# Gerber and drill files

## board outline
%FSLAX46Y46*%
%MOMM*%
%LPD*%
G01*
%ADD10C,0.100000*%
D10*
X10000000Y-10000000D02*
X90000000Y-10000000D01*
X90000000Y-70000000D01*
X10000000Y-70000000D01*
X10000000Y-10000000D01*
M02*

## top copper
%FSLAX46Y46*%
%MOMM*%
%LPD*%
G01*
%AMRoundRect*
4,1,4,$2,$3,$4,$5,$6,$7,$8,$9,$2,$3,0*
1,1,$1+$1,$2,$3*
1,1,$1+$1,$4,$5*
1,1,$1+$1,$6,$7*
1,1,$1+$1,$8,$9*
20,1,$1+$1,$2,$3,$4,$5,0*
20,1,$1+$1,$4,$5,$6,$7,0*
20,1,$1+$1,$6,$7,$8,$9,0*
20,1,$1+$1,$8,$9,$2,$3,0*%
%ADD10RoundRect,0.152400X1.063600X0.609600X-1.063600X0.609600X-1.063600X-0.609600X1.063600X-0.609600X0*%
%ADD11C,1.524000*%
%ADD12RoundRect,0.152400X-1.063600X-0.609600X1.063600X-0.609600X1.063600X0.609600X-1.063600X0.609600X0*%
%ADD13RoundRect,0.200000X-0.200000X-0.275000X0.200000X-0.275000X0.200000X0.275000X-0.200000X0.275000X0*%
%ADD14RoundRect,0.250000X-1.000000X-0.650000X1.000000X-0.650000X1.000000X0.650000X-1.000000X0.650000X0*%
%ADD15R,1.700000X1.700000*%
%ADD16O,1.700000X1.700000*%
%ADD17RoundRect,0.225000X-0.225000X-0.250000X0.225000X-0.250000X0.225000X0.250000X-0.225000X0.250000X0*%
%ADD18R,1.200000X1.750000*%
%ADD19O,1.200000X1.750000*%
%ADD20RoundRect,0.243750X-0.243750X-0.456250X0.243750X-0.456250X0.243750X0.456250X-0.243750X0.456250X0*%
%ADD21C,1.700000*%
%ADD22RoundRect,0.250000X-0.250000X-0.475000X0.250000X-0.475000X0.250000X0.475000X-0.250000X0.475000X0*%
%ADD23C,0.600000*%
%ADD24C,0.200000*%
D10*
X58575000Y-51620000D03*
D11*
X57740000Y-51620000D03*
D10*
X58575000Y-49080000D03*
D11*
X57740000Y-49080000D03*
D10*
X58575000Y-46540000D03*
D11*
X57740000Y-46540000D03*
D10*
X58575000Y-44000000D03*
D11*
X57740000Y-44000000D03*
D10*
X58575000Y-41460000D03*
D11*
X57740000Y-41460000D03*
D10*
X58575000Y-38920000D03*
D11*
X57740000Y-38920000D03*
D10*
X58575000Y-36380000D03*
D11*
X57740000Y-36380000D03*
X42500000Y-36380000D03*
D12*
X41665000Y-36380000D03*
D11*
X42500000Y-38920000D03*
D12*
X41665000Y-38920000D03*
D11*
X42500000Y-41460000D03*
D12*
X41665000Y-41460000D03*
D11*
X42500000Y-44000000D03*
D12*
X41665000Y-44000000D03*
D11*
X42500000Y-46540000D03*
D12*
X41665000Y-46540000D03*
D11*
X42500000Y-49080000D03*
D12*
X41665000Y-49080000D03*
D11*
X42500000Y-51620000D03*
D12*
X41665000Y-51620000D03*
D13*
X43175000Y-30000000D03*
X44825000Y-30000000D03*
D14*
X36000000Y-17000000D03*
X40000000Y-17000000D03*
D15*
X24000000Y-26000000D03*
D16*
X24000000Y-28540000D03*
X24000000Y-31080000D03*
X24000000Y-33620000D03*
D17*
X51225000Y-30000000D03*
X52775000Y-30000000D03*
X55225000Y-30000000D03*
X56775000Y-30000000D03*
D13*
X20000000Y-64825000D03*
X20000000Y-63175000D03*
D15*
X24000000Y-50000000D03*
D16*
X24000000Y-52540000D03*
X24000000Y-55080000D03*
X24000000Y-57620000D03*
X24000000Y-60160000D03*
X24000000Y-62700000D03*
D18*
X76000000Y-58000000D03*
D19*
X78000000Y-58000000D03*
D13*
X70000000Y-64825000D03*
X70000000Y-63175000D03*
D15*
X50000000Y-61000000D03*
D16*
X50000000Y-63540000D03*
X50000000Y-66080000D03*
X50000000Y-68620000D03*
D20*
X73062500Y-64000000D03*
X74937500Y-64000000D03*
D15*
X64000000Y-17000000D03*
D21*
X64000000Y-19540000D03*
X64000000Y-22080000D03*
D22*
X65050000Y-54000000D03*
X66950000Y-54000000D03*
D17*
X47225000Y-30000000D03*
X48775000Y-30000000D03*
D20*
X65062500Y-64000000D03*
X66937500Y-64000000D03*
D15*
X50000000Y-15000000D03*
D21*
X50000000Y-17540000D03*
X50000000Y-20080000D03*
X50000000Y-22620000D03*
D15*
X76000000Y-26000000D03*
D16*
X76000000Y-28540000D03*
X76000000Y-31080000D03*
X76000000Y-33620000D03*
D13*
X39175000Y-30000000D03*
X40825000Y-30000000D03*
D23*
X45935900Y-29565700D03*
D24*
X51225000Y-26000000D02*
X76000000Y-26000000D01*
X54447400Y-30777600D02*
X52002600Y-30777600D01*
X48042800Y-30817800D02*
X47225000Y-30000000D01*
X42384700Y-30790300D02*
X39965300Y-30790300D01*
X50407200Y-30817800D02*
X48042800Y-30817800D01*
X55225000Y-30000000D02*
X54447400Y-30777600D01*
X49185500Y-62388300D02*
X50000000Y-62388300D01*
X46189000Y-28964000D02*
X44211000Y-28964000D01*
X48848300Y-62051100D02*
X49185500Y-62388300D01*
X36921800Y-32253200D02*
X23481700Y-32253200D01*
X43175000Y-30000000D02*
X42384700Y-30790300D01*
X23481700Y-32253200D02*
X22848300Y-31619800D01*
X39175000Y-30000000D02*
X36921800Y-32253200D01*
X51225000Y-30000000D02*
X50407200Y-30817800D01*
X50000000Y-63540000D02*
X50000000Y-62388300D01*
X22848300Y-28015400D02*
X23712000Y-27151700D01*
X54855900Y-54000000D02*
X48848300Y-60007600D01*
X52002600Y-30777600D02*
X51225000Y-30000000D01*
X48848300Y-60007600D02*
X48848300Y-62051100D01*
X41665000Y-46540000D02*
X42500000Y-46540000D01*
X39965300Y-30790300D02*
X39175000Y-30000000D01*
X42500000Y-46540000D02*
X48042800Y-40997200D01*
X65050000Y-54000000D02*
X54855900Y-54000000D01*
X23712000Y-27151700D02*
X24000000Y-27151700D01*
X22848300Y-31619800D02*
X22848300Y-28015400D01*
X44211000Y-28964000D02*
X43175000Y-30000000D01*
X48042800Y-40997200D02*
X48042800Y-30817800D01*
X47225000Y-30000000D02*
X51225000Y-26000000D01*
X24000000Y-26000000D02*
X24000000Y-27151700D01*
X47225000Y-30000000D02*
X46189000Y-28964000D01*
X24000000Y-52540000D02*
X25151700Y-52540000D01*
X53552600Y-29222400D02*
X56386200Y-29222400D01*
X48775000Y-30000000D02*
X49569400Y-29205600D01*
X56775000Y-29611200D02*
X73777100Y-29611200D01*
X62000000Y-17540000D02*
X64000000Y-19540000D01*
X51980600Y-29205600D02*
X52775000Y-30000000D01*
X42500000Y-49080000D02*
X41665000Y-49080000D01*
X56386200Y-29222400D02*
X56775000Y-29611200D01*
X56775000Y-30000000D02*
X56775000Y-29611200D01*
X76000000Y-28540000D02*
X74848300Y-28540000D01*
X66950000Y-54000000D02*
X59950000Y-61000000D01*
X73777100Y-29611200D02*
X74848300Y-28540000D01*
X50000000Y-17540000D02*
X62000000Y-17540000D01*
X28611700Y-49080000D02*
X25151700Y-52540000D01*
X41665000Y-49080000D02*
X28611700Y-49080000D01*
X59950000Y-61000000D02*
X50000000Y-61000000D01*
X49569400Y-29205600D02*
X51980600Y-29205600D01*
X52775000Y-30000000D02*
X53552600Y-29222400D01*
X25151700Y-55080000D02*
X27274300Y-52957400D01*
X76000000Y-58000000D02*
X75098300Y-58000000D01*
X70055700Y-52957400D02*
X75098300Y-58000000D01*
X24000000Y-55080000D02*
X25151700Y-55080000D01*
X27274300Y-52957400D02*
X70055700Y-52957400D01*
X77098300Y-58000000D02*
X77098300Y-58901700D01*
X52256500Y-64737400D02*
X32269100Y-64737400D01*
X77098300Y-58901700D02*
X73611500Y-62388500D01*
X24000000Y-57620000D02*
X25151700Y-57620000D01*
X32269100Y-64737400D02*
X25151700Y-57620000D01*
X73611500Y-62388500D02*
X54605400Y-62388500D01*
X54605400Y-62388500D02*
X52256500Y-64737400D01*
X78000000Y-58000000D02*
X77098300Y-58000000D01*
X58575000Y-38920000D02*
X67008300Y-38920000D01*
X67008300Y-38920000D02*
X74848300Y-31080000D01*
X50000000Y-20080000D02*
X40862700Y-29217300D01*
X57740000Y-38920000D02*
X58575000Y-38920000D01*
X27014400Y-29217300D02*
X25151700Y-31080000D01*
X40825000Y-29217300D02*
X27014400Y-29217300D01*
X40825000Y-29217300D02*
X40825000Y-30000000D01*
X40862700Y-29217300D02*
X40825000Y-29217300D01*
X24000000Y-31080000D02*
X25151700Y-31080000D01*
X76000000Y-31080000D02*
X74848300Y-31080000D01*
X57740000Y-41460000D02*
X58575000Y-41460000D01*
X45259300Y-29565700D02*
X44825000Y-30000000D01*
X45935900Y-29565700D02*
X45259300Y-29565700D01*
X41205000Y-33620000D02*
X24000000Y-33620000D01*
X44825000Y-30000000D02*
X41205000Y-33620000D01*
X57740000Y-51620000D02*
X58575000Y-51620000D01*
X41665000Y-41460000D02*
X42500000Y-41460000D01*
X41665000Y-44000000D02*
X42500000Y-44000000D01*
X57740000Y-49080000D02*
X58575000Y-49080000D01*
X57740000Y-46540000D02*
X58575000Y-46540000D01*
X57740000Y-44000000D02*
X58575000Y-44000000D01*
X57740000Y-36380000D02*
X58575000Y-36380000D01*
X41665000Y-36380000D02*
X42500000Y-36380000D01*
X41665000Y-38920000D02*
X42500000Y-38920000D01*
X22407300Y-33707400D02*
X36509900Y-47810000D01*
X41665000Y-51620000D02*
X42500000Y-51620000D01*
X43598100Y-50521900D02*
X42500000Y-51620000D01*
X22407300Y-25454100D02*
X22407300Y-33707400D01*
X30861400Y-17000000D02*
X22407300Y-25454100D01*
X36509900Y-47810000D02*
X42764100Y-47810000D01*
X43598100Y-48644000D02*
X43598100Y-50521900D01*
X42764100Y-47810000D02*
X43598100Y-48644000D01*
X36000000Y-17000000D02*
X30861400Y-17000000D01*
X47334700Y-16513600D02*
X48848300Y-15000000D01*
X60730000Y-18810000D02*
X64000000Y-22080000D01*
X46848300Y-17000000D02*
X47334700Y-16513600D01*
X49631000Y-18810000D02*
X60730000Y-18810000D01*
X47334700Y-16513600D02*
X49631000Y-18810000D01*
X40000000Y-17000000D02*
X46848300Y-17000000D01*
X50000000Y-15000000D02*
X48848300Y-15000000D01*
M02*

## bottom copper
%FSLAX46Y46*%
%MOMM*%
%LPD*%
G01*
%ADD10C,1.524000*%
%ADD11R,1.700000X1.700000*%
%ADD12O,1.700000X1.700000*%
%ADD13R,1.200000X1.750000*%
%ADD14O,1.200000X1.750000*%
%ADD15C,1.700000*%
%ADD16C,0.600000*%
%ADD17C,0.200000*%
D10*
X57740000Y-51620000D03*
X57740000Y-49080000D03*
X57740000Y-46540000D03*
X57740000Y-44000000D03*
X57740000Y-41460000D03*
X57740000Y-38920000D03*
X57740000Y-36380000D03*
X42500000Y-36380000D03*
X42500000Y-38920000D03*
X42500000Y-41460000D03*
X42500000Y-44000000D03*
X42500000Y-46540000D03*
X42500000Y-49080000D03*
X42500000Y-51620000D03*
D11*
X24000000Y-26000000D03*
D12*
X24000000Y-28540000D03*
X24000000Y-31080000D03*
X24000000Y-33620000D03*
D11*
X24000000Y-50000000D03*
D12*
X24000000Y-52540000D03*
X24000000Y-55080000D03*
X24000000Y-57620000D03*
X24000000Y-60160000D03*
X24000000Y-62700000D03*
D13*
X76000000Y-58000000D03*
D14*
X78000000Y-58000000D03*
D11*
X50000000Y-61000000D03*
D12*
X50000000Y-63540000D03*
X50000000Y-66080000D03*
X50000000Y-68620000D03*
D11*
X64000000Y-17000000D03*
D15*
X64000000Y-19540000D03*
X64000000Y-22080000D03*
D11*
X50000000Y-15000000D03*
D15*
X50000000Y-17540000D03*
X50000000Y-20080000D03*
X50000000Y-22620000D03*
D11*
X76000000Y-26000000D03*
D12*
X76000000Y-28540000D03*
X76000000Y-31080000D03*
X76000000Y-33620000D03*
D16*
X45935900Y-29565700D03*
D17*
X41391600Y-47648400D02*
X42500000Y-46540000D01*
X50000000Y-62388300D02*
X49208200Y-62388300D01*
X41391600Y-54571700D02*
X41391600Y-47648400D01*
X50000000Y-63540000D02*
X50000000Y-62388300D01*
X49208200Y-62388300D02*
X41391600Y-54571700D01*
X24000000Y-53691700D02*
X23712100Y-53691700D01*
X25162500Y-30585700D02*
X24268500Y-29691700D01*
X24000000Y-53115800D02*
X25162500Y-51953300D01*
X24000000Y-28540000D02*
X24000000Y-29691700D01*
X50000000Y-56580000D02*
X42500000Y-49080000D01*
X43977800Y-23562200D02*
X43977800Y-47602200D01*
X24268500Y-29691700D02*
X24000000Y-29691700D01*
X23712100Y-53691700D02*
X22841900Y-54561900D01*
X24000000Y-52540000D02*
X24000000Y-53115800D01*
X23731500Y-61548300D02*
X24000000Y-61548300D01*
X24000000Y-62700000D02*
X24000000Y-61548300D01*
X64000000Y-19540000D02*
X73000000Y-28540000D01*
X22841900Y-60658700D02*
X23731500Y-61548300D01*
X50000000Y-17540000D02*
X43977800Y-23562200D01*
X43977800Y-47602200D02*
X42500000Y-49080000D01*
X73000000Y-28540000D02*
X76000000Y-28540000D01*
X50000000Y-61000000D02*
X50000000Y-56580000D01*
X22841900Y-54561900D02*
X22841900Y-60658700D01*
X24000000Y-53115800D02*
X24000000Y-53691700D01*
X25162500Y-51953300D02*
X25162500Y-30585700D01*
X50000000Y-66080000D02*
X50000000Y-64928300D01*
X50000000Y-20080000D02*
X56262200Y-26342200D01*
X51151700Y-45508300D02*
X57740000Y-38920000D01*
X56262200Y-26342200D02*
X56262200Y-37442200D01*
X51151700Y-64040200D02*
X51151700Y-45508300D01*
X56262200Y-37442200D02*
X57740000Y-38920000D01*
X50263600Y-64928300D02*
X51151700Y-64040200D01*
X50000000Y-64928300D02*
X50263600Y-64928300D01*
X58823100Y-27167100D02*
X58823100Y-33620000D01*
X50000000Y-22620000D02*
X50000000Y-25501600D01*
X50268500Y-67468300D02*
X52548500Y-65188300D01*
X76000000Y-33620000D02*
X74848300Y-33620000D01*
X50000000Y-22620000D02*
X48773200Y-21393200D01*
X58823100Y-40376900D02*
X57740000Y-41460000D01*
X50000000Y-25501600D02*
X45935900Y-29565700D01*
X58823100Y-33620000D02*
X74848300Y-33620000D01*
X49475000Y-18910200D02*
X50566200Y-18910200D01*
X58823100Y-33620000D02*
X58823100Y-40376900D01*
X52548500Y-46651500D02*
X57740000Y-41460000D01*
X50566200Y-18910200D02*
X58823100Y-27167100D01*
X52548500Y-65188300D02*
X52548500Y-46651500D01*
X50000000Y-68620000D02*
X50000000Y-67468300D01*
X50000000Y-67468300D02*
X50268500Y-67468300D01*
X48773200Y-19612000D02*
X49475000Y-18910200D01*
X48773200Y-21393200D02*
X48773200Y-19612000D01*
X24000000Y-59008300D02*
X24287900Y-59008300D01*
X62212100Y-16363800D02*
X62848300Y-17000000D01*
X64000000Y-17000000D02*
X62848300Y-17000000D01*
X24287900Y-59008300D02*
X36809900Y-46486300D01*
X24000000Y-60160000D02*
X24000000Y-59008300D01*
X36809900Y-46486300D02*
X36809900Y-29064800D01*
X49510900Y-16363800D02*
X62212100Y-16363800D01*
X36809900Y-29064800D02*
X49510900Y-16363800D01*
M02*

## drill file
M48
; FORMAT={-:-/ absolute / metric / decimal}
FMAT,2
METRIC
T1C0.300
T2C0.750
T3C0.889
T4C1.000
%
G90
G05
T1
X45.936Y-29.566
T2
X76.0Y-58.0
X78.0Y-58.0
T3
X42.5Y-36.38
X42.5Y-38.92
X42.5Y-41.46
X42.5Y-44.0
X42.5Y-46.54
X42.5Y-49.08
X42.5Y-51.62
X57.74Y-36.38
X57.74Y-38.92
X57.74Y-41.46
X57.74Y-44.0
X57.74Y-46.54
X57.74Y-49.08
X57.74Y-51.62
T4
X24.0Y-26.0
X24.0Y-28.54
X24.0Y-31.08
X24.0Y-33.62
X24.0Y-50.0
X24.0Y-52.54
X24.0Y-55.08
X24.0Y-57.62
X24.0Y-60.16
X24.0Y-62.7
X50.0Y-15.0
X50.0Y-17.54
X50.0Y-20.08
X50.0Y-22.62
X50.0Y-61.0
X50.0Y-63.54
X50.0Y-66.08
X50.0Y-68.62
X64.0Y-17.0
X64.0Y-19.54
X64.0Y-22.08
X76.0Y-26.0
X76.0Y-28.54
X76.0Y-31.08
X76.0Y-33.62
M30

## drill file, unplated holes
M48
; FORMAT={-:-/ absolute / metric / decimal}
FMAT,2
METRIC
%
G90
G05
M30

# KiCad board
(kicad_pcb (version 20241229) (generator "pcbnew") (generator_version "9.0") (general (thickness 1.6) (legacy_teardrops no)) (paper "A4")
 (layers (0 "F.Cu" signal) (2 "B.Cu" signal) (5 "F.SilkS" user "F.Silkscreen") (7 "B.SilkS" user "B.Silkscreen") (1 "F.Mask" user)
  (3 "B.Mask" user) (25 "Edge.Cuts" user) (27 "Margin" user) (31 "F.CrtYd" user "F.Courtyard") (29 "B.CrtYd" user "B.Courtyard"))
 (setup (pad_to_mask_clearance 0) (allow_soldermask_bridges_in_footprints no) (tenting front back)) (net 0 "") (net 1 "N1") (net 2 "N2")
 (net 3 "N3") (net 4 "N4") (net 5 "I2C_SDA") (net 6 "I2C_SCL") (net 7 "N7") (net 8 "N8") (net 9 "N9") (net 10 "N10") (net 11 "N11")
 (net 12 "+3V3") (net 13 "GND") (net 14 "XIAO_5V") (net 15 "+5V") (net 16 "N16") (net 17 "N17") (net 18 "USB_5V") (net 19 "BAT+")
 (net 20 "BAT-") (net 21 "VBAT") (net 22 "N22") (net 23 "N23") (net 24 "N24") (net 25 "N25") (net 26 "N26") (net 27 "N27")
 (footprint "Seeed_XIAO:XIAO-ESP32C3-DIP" (layer "F.Cu") (at 50 44 180)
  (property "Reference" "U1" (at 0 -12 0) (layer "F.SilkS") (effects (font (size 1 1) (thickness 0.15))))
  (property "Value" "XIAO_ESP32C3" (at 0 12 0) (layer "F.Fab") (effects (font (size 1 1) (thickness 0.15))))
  (pad "1" smd roundrect (at -8.575 -7.62 180) (size 2.432 1.524) (layers "F.Cu" "F.Mask") (roundrect_rratio 0.1) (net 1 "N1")
   (thermal_bridge_angle 45))
  (pad "1" thru_hole circle (at -7.74 -7.62 180) (size 1.524 1.524) (drill 0.889) (layers "*.Cu" "*.Mask") (remove_unused_layers no)
   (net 1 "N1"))
  (pad "2" smd roundrect (at -8.575 -5.08 180) (size 2.432 1.524) (layers "F.Cu" "F.Mask") (roundrect_rratio 0.1) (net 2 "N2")
   (thermal_bridge_angle 45))
  (pad "2" thru_hole circle (at -7.74 -5.08 180) (size 1.524 1.524) (drill 0.889) (layers "*.Cu" "*.Mask") (remove_unused_layers no)
   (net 2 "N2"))
  (pad "3" smd roundrect (at -8.575 -2.54 180) (size 2.432 1.524) (layers "F.Cu" "F.Mask") (roundrect_rratio 0.1) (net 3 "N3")
   (thermal_bridge_angle 45))
  (pad "3" thru_hole circle (at -7.74 -2.54 180) (size 1.524 1.524) (drill 0.889) (layers "*.Cu" "*.Mask") (remove_unused_layers no)
   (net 3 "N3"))
  (pad "4" smd roundrect (at -8.575 0 180) (size 2.432 1.524) (layers "F.Cu" "F.Mask") (roundrect_rratio 0.1) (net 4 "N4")
   (thermal_bridge_angle 45))
  (pad "4" thru_hole circle (at -7.74 0 180) (size 1.524 1.524) (drill 0.889) (layers "*.Cu" "*.Mask") (remove_unused_layers no)
   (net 4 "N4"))
  (pad "5" smd roundrect (at -8.575 2.54 180) (size 2.432 1.524) (layers "F.Cu" "F.Mask") (roundrect_rratio 0.1) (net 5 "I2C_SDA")
   (thermal_bridge_angle 45))
  (pad "5" thru_hole circle (at -7.74 2.54 180) (size 1.524 1.524) (drill 0.889) (layers "*.Cu" "*.Mask") (remove_unused_layers no)
   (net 5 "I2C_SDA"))
  (pad "6" smd roundrect (at -8.575 5.08 180) (size 2.432 1.524) (layers "F.Cu" "F.Mask") (roundrect_rratio 0.1) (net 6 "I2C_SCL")
   (thermal_bridge_angle 45))
  (pad "6" thru_hole circle (at -7.74 5.08 180) (size 1.524 1.524) (drill 0.889) (layers "*.Cu" "*.Mask") (remove_unused_layers no)
   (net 6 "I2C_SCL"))
  (pad "7" smd roundrect (at -8.575 7.62 180) (size 2.432 1.524) (layers "F.Cu" "F.Mask") (roundrect_rratio 0.1) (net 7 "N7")
   (thermal_bridge_angle 45))
  (pad "7" thru_hole circle (at -7.74 7.62 180) (size 1.524 1.524) (drill 0.889) (layers "*.Cu" "*.Mask") (remove_unused_layers no)
   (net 7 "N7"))
  (pad "8" thru_hole circle (at 7.5 7.62) (size 1.524 1.524) (drill 0.889) (layers "*.Cu" "*.Mask") (remove_unused_layers no) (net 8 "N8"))
  (pad "8" smd roundrect (at 8.335 7.62) (size 2.432 1.524) (layers "F.Cu" "F.Mask") (roundrect_rratio 0.1) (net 8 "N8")
   (thermal_bridge_angle 45))
  (pad "9" thru_hole circle (at 7.5 5.08) (size 1.524 1.524) (drill 0.889) (layers "*.Cu" "*.Mask") (remove_unused_layers no) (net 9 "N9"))
  (pad "9" smd roundrect (at 8.335 5.08) (size 2.432 1.524) (layers "F.Cu" "F.Mask") (roundrect_rratio 0.1) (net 9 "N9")
   (thermal_bridge_angle 45))
  (pad "10" thru_hole circle (at 7.5 2.54) (size 1.524 1.524) (drill 0.889) (layers "*.Cu" "*.Mask") (remove_unused_layers no)
   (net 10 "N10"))
  (pad "10" smd roundrect (at 8.335 2.54) (size 2.432 1.524) (layers "F.Cu" "F.Mask") (roundrect_rratio 0.1) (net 10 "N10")
   (thermal_bridge_angle 45))
  (pad "11" thru_hole circle (at 7.5 0) (size 1.524 1.524) (drill 0.889) (layers "*.Cu" "*.Mask") (remove_unused_layers no) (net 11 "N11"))
  (pad "11" smd roundrect (at 8.335 0) (size 2.432 1.524) (layers "F.Cu" "F.Mask") (roundrect_rratio 0.1) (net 11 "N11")
   (thermal_bridge_angle 45))
  (pad "12" thru_hole circle (at 7.5 -2.54) (size 1.524 1.524) (drill 0.889) (layers "*.Cu" "*.Mask") (remove_unused_layers no)
   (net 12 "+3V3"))
  (pad "12" smd roundrect (at 8.335 -2.54) (size 2.432 1.524) (layers "F.Cu" "F.Mask") (roundrect_rratio 0.1) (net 12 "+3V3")
   (thermal_bridge_angle 45))
  (pad "13" thru_hole circle (at 7.5 -5.08) (size 1.524 1.524) (drill 0.889) (layers "*.Cu" "*.Mask") (remove_unused_layers no)
   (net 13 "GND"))
  (pad "13" smd roundrect (at 8.335 -5.08) (size 2.432 1.524) (layers "F.Cu" "F.Mask") (roundrect_rratio 0.1) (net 13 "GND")
   (thermal_bridge_angle 45))
  (pad "14" thru_hole circle (at 7.5 -7.62) (size 1.524 1.524) (drill 0.889) (layers "*.Cu" "*.Mask") (remove_unused_layers no)
   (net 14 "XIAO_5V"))
  (pad "14" smd roundrect (at 8.335 -7.62) (size 2.432 1.524) (layers "F.Cu" "F.Mask") (roundrect_rratio 0.1) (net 14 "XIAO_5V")
   (thermal_bridge_angle 45)))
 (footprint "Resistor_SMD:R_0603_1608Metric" (layer "F.Cu") (at 44 30)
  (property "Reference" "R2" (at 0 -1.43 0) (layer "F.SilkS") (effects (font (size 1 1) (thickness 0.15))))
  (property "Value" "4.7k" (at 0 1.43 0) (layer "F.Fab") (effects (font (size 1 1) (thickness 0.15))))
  (pad "1" smd roundrect (at -0.825 0) (size 0.8 0.95) (layers "F.Cu" "F.Mask" "F.Paste") (roundrect_rratio 0.25) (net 12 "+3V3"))
  (pad "2" smd roundrect (at 0.825 0) (size 0.8 0.95) (layers "F.Cu" "F.Mask" "F.Paste") (roundrect_rratio 0.25) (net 5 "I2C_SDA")))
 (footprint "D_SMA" (layer "F.Cu") (at 38 17)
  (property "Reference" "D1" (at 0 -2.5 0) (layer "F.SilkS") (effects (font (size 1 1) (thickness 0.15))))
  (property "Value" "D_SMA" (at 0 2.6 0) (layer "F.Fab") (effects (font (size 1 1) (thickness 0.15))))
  (pad "1" smd roundrect (at -2 0) (size 2.5 1.8) (layers "F.Cu" "F.Mask" "F.Paste") (roundrect_rratio 0.1388888889) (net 14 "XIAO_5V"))
  (pad "2" smd roundrect (at 2 0) (size 2.5 1.8) (layers "F.Cu" "F.Mask" "F.Paste") (roundrect_rratio 0.1388888889) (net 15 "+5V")))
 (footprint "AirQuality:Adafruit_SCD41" (layer "F.Cu") (at 24 26)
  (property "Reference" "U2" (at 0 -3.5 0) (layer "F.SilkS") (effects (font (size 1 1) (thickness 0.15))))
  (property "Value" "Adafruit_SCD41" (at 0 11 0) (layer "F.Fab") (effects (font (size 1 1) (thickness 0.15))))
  (pad "1" thru_hole rect (at 0 0) (size 1.7 1.7) (drill 1) (layers "*.Cu" "*.Mask") (remove_unused_layers no) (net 12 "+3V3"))
  (pad "2" thru_hole oval (at 0 2.54) (size 1.7 1.7) (drill 1) (layers "*.Cu" "*.Mask") (remove_unused_layers no) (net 13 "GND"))
  (pad "3" thru_hole oval (at 0 5.08) (size 1.7 1.7) (drill 1) (layers "*.Cu" "*.Mask") (remove_unused_layers no) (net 6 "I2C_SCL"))
  (pad "4" thru_hole oval (at 0 7.62) (size 1.7 1.7) (drill 1) (layers "*.Cu" "*.Mask") (remove_unused_layers no) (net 5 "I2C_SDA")))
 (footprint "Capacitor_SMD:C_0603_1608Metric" (layer "F.Cu") (at 52 30)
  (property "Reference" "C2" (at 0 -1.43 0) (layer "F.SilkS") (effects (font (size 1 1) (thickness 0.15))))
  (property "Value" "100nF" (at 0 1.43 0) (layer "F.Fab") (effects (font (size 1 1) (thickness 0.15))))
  (pad "1" smd roundrect (at -0.775 0) (size 0.9 0.95) (layers "F.Cu" "F.Mask" "F.Paste") (roundrect_rratio 0.25) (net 12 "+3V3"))
  (pad "2" smd roundrect (at 0.775 0) (size 0.9 0.95) (layers "F.Cu" "F.Mask" "F.Paste") (roundrect_rratio 0.25) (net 13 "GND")))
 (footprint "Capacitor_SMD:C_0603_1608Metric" (layer "F.Cu") (at 56 30)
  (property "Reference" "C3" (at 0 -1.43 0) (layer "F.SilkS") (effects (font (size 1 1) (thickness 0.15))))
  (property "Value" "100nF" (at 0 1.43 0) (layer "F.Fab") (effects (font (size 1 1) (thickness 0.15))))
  (pad "1" smd roundrect (at -0.775 0) (size 0.9 0.95) (layers "F.Cu" "F.Mask" "F.Paste") (roundrect_rratio 0.25) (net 12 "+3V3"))
  (pad "2" smd roundrect (at 0.775 0) (size 0.9 0.95) (layers "F.Cu" "F.Mask" "F.Paste") (roundrect_rratio 0.25) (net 13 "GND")))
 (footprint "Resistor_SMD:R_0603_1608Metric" (layer "F.Cu") (at 20 64 90)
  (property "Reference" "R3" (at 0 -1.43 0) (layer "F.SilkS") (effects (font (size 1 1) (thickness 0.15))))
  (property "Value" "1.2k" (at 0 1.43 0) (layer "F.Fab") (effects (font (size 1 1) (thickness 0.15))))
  (pad "1" smd roundrect (at -0.825 0) (size 0.8 0.95) (layers "F.Cu" "F.Mask" "F.Paste") (roundrect_rratio 0.25) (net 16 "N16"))
  (pad "2" smd roundrect (at 0.825 0) (size 0.8 0.95) (layers "F.Cu" "F.Mask" "F.Paste") (roundrect_rratio 0.25) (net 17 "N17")))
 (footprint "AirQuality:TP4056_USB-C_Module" (layer "F.Cu") (at 24 50)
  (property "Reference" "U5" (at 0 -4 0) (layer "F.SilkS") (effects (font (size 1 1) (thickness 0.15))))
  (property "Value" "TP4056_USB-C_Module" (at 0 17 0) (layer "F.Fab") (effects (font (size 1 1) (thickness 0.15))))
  (pad "1" thru_hole rect (at 0 0) (size 1.7 1.7) (drill 1) (layers "*.Cu" "*.Mask") (remove_unused_layers no) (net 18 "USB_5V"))
  (pad "2" thru_hole oval (at 0 2.54) (size 1.7 1.7) (drill 1) (layers "*.Cu" "*.Mask") (remove_unused_layers no) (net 13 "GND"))
  (pad "3" thru_hole oval (at 0 5.08) (size 1.7 1.7) (drill 1) (layers "*.Cu" "*.Mask") (remove_unused_layers no) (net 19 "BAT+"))
  (pad "4" thru_hole oval (at 0 7.62) (size 1.7 1.7) (drill 1) (layers "*.Cu" "*.Mask") (remove_unused_layers no) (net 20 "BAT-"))
  (pad "5" thru_hole oval (at 0 10.16) (size 1.7 1.7) (drill 1) (layers "*.Cu" "*.Mask") (remove_unused_layers no) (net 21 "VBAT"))
  (pad "6" thru_hole oval (at 0 12.7) (size 1.7 1.7) (drill 1) (layers "*.Cu" "*.Mask") (remove_unused_layers no) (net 13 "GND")))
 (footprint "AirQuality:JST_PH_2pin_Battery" (layer "F.Cu") (at 76 58)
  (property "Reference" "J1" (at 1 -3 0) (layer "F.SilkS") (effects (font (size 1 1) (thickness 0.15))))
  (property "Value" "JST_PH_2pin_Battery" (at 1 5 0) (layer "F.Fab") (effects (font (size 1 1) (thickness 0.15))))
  (pad "1" thru_hole rect (at 0 0) (size 1.2 1.75) (drill 0.75) (layers "*.Cu" "*.Mask") (remove_unused_layers no) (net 19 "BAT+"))
  (pad "2" thru_hole oval (at 2 0) (size 1.2 1.75) (drill 0.75) (layers "*.Cu" "*.Mask") (remove_unused_layers no) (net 20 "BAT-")))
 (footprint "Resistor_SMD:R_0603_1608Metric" (layer "F.Cu") (at 70 64 90)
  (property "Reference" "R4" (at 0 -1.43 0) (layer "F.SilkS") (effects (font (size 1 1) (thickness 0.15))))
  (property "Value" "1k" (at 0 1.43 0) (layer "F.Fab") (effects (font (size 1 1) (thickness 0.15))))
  (pad "1" smd roundrect (at -0.825 0) (size 0.8 0.95) (layers "F.Cu" "F.Mask" "F.Paste") (roundrect_rratio 0.25) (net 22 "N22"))
  (pad "2" smd roundrect (at 0.825 0) (size 0.8 0.95) (layers "F.Cu" "F.Mask" "F.Paste") (roundrect_rratio 0.25) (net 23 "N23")))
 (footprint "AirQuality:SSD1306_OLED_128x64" (layer "F.Cu") (at 50 61)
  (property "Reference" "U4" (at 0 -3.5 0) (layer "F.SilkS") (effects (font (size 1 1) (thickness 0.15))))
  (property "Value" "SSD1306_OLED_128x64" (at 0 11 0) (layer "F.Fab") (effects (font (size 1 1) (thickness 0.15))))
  (pad "1" thru_hole rect (at 0 0) (size 1.7 1.7) (drill 1) (layers "*.Cu" "*.Mask") (remove_unused_layers no) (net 13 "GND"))
  (pad "2" thru_hole oval (at 0 2.54) (size 1.7 1.7) (drill 1) (layers "*.Cu" "*.Mask") (remove_unused_layers no) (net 12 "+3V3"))
  (pad "3" thru_hole oval (at 0 5.08) (size 1.7 1.7) (drill 1) (layers "*.Cu" "*.Mask") (remove_unused_layers no) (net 6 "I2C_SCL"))
  (pad "4" thru_hole oval (at 0 7.62) (size 1.7 1.7) (drill 1) (layers "*.Cu" "*.Mask") (remove_unused_layers no) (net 5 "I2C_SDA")))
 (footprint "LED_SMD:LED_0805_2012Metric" (layer "F.Cu") (at 74 64)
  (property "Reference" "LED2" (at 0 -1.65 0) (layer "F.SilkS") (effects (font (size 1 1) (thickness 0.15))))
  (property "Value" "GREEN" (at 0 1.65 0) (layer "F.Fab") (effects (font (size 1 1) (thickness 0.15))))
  (pad "1" smd roundrect (at -0.9375 0) (size 0.975 1.4) (layers "F.Cu" "F.Mask" "F.Paste") (roundrect_rratio 0.25) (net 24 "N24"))
  (pad "2" smd roundrect (at 0.9375 0) (size 0.975 1.4) (layers "F.Cu" "F.Mask" "F.Paste") (roundrect_rratio 0.25) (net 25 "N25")))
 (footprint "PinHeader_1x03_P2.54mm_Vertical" (layer "F.Cu") (at 64 17)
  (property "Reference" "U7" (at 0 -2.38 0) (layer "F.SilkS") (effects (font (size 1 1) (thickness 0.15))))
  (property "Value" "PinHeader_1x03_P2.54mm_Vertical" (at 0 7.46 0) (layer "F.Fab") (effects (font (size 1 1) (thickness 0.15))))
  (pad "1" thru_hole rect (at 0 0) (size 1.7 1.7) (drill 1) (layers "*.Cu" "*.Mask") (remove_unused_layers no) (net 21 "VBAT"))
  (pad "2" thru_hole circle (at 0 2.54) (size 1.7 1.7) (drill 1) (layers "*.Cu" "*.Mask") (remove_unused_layers no) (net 13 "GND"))
  (pad "3" thru_hole circle (at 0 5.08) (size 1.7 1.7) (drill 1) (layers "*.Cu" "*.Mask") (remove_unused_layers no) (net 15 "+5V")))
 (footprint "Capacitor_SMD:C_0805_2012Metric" (layer "F.Cu") (at 66 54)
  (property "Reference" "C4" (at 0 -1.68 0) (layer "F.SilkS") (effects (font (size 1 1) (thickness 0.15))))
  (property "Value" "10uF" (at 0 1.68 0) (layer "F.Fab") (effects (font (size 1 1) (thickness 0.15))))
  (pad "1" smd roundrect (at -0.95 0) (size 1 1.45) (layers "F.Cu" "F.Mask" "F.Paste") (roundrect_rratio 0.25) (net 12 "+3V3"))
  (pad "2" smd roundrect (at 0.95 0) (size 1 1.45) (layers "F.Cu" "F.Mask" "F.Paste") (roundrect_rratio 0.25) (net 13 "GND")))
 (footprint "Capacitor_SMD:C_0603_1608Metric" (layer "F.Cu") (at 48 30)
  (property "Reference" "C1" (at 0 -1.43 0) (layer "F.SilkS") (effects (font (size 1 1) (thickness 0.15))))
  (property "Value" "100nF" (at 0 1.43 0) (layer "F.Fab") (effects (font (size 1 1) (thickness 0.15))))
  (pad "1" smd roundrect (at -0.775 0) (size 0.9 0.95) (layers "F.Cu" "F.Mask" "F.Paste") (roundrect_rratio 0.25) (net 12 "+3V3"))
  (pad "2" smd roundrect (at 0.775 0) (size 0.9 0.95) (layers "F.Cu" "F.Mask" "F.Paste") (roundrect_rratio 0.25) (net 13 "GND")))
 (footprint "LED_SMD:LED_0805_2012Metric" (layer "F.Cu") (at 66 64)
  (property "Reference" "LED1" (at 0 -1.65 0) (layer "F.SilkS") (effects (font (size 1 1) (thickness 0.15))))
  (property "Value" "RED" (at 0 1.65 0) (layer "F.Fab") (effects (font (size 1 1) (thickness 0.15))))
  (pad "1" smd roundrect (at -0.9375 0) (size 0.975 1.4) (layers "F.Cu" "F.Mask" "F.Paste") (roundrect_rratio 0.25) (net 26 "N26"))
  (pad "2" smd roundrect (at 0.9375 0) (size 0.975 1.4) (layers "F.Cu" "F.Mask" "F.Paste") (roundrect_rratio 0.25) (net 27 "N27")))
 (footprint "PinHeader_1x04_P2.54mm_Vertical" (layer "F.Cu") (at 50 15)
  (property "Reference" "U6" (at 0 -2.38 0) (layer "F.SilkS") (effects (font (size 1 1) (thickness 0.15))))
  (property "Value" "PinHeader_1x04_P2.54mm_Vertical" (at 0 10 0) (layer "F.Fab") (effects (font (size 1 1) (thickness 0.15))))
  (pad "1" thru_hole rect (at 0 0) (size 1.7 1.7) (drill 1) (layers "*.Cu" "*.Mask") (remove_unused_layers no) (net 15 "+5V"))
  (pad "2" thru_hole circle (at 0 2.54) (size 1.7 1.7) (drill 1) (layers "*.Cu" "*.Mask") (remove_unused_layers no) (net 13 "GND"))
  (pad "3" thru_hole circle (at 0 5.08) (size 1.7 1.7) (drill 1) (layers "*.Cu" "*.Mask") (remove_unused_layers no) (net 6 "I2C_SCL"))
  (pad "4" thru_hole circle (at 0 7.62) (size 1.7 1.7) (drill 1) (layers "*.Cu" "*.Mask") (remove_unused_layers no) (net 5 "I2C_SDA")))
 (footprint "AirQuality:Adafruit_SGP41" (layer "F.Cu") (at 76 26)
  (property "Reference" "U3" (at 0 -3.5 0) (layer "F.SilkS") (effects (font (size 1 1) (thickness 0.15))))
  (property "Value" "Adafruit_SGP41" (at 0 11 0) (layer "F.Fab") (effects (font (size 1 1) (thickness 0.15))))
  (pad "1" thru_hole rect (at 0 0) (size 1.7 1.7) (drill 1) (layers "*.Cu" "*.Mask") (remove_unused_layers no) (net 12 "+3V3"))
  (pad "2" thru_hole oval (at 0 2.54) (size 1.7 1.7) (drill 1) (layers "*.Cu" "*.Mask") (remove_unused_layers no) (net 13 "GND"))
  (pad "3" thru_hole oval (at 0 5.08) (size 1.7 1.7) (drill 1) (layers "*.Cu" "*.Mask") (remove_unused_layers no) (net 6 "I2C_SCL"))
  (pad "4" thru_hole oval (at 0 7.62) (size 1.7 1.7) (drill 1) (layers "*.Cu" "*.Mask") (remove_unused_layers no) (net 5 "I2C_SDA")))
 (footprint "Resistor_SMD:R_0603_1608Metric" (layer "F.Cu") (at 40 30)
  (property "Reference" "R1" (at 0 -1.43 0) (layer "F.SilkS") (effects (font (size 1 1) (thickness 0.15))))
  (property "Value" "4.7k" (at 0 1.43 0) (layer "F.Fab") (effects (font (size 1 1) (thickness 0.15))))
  (pad "1" smd roundrect (at -0.825 0) (size 0.8 0.95) (layers "F.Cu" "F.Mask" "F.Paste") (roundrect_rratio 0.25) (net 12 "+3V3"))
  (pad "2" smd roundrect (at 0.825 0) (size 0.8 0.95) (layers "F.Cu" "F.Mask" "F.Paste") (roundrect_rratio 0.25) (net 6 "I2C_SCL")))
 (gr_rect (start 10 10) (end 90 70) (stroke (width 0.1) (type solid)) (fill no) (layer "Edge.Cuts"))
 (segment (start 51.225 26) (end 76 26) (width 0.2) (layer "F.Cu") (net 12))
 (segment (start 54.4474 30.7776) (end 52.0026 30.7776) (width 0.2) (layer "F.Cu") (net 12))
 (segment (start 48.0428 30.8178) (end 47.225 30) (width 0.2) (layer "F.Cu") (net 12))
 (segment (start 42.3847 30.7903) (end 39.9653 30.7903) (width 0.2) (layer "F.Cu") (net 12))
 (segment (start 50.4072 30.8178) (end 48.0428 30.8178) (width 0.2) (layer "F.Cu") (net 12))
 (segment (start 55.225 30) (end 54.4474 30.7776) (width 0.2) (layer "F.Cu") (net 12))
 (segment (start 49.1855 62.3883) (end 50 62.3883) (width 0.2) (layer "F.Cu") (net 12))
 (segment (start 46.189 28.964) (end 44.211 28.964) (width 0.2) (layer "F.Cu") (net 12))
 (segment (start 48.8483 62.0511) (end 49.1855 62.3883) (width 0.2) (layer "F.Cu") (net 12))
 (segment (start 36.9218 32.2532) (end 23.4817 32.2532) (width 0.2) (layer "F.Cu") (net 12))
 (segment (start 43.175 30) (end 42.3847 30.7903) (width 0.2) (layer "F.Cu") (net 12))
 (segment (start 23.4817 32.2532) (end 22.8483 31.6198) (width 0.2) (layer "F.Cu") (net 12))
 (segment (start 39.175 30) (end 36.9218 32.2532) (width 0.2) (layer "F.Cu") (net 12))
 (segment (start 51.225 30) (end 50.4072 30.8178) (width 0.2) (layer "F.Cu") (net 12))
 (segment (start 50 63.54) (end 50 62.3883) (width 0.2) (layer "F.Cu") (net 12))
 (segment (start 22.8483 28.0154) (end 23.712 27.1517) (width 0.2) (layer "F.Cu") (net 12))
 (segment (start 54.8559 54) (end 48.8483 60.0076) (width 0.2) (layer "F.Cu") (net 12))
 (segment (start 52.0026 30.7776) (end 51.225 30) (width 0.2) (layer "F.Cu") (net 12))
 (segment (start 48.8483 60.0076) (end 48.8483 62.0511) (width 0.2) (layer "F.Cu") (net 12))
 (segment (start 41.665 46.54) (end 42.5 46.54) (width 0.2) (layer "F.Cu") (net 12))
 (segment (start 39.9653 30.7903) (end 39.175 30) (width 0.2) (layer "F.Cu") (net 12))
 (segment (start 42.5 46.54) (end 48.0428 40.9972) (width 0.2) (layer "F.Cu") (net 12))
 (segment (start 65.05 54) (end 54.8559 54) (width 0.2) (layer "F.Cu") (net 12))
 (segment (start 23.712 27.1517) (end 24 27.1517) (width 0.2) (layer "F.Cu") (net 12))
 (segment (start 22.8483 31.6198) (end 22.8483 28.0154) (width 0.2) (layer "F.Cu") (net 12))
 (segment (start 44.211 28.964) (end 43.175 30) (width 0.2) (layer "F.Cu") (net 12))
 (segment (start 48.0428 40.9972) (end 48.0428 30.8178) (width 0.2) (layer "F.Cu") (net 12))
 (segment (start 47.225 30) (end 51.225 26) (width 0.2) (layer "F.Cu") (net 12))
 (segment (start 24 26) (end 24 27.1517) (width 0.2) (layer "F.Cu") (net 12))
 (segment (start 47.225 30) (end 46.189 28.964) (width 0.2) (layer "F.Cu") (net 12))
 (segment (start 41.3916 47.6484) (end 42.5 46.54) (width 0.2) (layer "B.Cu") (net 12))
 (segment (start 50 62.3883) (end 49.2082 62.3883) (width 0.2) (layer "B.Cu") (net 12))
 (segment (start 41.3916 54.5717) (end 41.3916 47.6484) (width 0.2) (layer "B.Cu") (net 12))
 (segment (start 50 63.54) (end 50 62.3883) (width 0.2) (layer "B.Cu") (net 12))
 (segment (start 49.2082 62.3883) (end 41.3916 54.5717) (width 0.2) (layer "B.Cu") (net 12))
 (segment (start 24 52.54) (end 25.1517 52.54) (width 0.2) (layer "F.Cu") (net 13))
 (segment (start 53.5526 29.2224) (end 56.3862 29.2224) (width 0.2) (layer "F.Cu") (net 13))
 (segment (start 48.775 30) (end 49.5694 29.2056) (width 0.2) (layer "F.Cu") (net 13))
 (segment (start 56.775 29.6112) (end 73.7771 29.6112) (width 0.2) (layer "F.Cu") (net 13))
 (segment (start 62 17.54) (end 64 19.54) (width 0.2) (layer "F.Cu") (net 13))
 (segment (start 51.9806 29.2056) (end 52.775 30) (width 0.2) (layer "F.Cu") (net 13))
 (segment (start 42.5 49.08) (end 41.665 49.08) (width 0.2) (layer "F.Cu") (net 13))
 (segment (start 56.3862 29.2224) (end 56.775 29.6112) (width 0.2) (layer "F.Cu") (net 13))
 (segment (start 56.775 30) (end 56.775 29.6112) (width 0.2) (layer "F.Cu") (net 13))
 (segment (start 76 28.54) (end 74.8483 28.54) (width 0.2) (layer "F.Cu") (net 13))
 (segment (start 66.95 54) (end 59.95 61) (width 0.2) (layer "F.Cu") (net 13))
 (segment (start 73.7771 29.6112) (end 74.8483 28.54) (width 0.2) (layer "F.Cu") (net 13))
 (segment (start 50 17.54) (end 62 17.54) (width 0.2) (layer "F.Cu") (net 13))
 (segment (start 28.6117 49.08) (end 25.1517 52.54) (width 0.2) (layer "F.Cu") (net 13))
 (segment (start 41.665 49.08) (end 28.6117 49.08) (width 0.2) (layer "F.Cu") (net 13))
 (segment (start 59.95 61) (end 50 61) (width 0.2) (layer "F.Cu") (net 13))
 (segment (start 49.5694 29.2056) (end 51.9806 29.2056) (width 0.2) (layer "F.Cu") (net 13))
 (segment (start 52.775 30) (end 53.5526 29.2224) (width 0.2) (layer "F.Cu") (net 13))
 (segment (start 24 53.6917) (end 23.7121 53.6917) (width 0.2) (layer "B.Cu") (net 13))
 (segment (start 25.1625 30.5857) (end 24.2685 29.6917) (width 0.2) (layer "B.Cu") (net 13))
 (segment (start 24 53.1158) (end 25.1625 51.9533) (width 0.2) (layer "B.Cu") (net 13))
 (segment (start 24 28.54) (end 24 29.6917) (width 0.2) (layer "B.Cu") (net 13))
 (segment (start 50 56.58) (end 42.5 49.08) (width 0.2) (layer "B.Cu") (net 13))
 (segment (start 43.9778 23.5622) (end 43.9778 47.6022) (width 0.2) (layer "B.Cu") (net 13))
 (segment (start 24.2685 29.6917) (end 24 29.6917) (width 0.2) (layer "B.Cu") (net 13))
 (segment (start 23.7121 53.6917) (end 22.8419 54.5619) (width 0.2) (layer "B.Cu") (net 13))
 (segment (start 24 52.54) (end 24 53.1158) (width 0.2) (layer "B.Cu") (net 13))
 (segment (start 23.7315 61.5483) (end 24 61.5483) (width 0.2) (layer "B.Cu") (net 13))
 (segment (start 24 62.7) (end 24 61.5483) (width 0.2) (layer "B.Cu") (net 13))
 (segment (start 64 19.54) (end 73 28.54) (width 0.2) (layer "B.Cu") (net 13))
 (segment (start 22.8419 60.6587) (end 23.7315 61.5483) (width 0.2) (layer "B.Cu") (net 13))
 (segment (start 50 17.54) (end 43.9778 23.5622) (width 0.2) (layer "B.Cu") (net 13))
 (segment (start 43.9778 47.6022) (end 42.5 49.08) (width 0.2) (layer "B.Cu") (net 13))
 (segment (start 73 28.54) (end 76 28.54) (width 0.2) (layer "B.Cu") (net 13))
 (segment (start 50 61) (end 50 56.58) (width 0.2) (layer "B.Cu") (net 13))
 (segment (start 22.8419 54.5619) (end 22.8419 60.6587) (width 0.2) (layer "B.Cu") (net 13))
 (segment (start 24 53.1158) (end 24 53.6917) (width 0.2) (layer "B.Cu") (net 13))
 (segment (start 25.1625 51.9533) (end 25.1625 30.5857) (width 0.2) (layer "B.Cu") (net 13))
 (segment (start 25.1517 55.08) (end 27.2743 52.9574) (width 0.2) (layer "F.Cu") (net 19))
 (segment (start 76 58) (end 75.0983 58) (width 0.2) (layer "F.Cu") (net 19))
 (segment (start 70.0557 52.9574) (end 75.0983 58) (width 0.2) (layer "F.Cu") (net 19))
 (segment (start 24 55.08) (end 25.1517 55.08) (width 0.2) (layer "F.Cu") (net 19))
 (segment (start 27.2743 52.9574) (end 70.0557 52.9574) (width 0.2) (layer "F.Cu") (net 19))
 (segment (start 77.0983 58) (end 77.0983 58.9017) (width 0.2) (layer "F.Cu") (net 20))
 (segment (start 52.2565 64.7374) (end 32.2691 64.7374) (width 0.2) (layer "F.Cu") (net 20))
 (segment (start 77.0983 58.9017) (end 73.6115 62.3885) (width 0.2) (layer "F.Cu") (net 20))
 (segment (start 24 57.62) (end 25.1517 57.62) (width 0.2) (layer "F.Cu") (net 20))
 (segment (start 32.2691 64.7374) (end 25.1517 57.62) (width 0.2) (layer "F.Cu") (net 20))
 (segment (start 73.6115 62.3885) (end 54.6054 62.3885) (width 0.2) (layer "F.Cu") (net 20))
 (segment (start 54.6054 62.3885) (end 52.2565 64.7374) (width 0.2) (layer "F.Cu") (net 20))
 (segment (start 78 58) (end 77.0983 58) (width 0.2) (layer "F.Cu") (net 20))
 (segment (start 58.575 38.92) (end 67.0083 38.92) (width 0.2) (layer "F.Cu") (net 6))
 (segment (start 67.0083 38.92) (end 74.8483 31.08) (width 0.2) (layer "F.Cu") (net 6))
 (segment (start 50 20.08) (end 40.8627 29.2173) (width 0.2) (layer "F.Cu") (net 6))
 (segment (start 57.74 38.92) (end 58.575 38.92) (width 0.2) (layer "F.Cu") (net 6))
 (segment (start 27.0144 29.2173) (end 25.1517 31.08) (width 0.2) (layer "F.Cu") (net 6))
 (segment (start 40.825 29.2173) (end 27.0144 29.2173) (width 0.2) (layer "F.Cu") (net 6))
 (segment (start 40.825 29.2173) (end 40.825 30) (width 0.2) (layer "F.Cu") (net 6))
 (segment (start 40.8627 29.2173) (end 40.825 29.2173) (width 0.2) (layer "F.Cu") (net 6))
 (segment (start 24 31.08) (end 25.1517 31.08) (width 0.2) (layer "F.Cu") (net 6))
 (segment (start 76 31.08) (end 74.8483 31.08) (width 0.2) (layer "F.Cu") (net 6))
 (segment (start 50 66.08) (end 50 64.9283) (width 0.2) (layer "B.Cu") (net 6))
 (segment (start 50 20.08) (end 56.2622 26.3422) (width 0.2) (layer "B.Cu") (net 6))
 (segment (start 51.1517 45.5083) (end 57.74 38.92) (width 0.2) (layer "B.Cu") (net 6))
 (segment (start 56.2622 26.3422) (end 56.2622 37.4422) (width 0.2) (layer "B.Cu") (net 6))
 (segment (start 51.1517 64.0402) (end 51.1517 45.5083) (width 0.2) (layer "B.Cu") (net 6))
 (segment (start 56.2622 37.4422) (end 57.74 38.92) (width 0.2) (layer "B.Cu") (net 6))
 (segment (start 50.2636 64.9283) (end 51.1517 64.0402) (width 0.2) (layer "B.Cu") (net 6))
 (segment (start 50 64.9283) (end 50.2636 64.9283) (width 0.2) (layer "B.Cu") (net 6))
 (segment (start 57.74 41.46) (end 58.575 41.46) (width 0.2) (layer "F.Cu") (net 5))
 (segment (start 45.2593 29.5657) (end 44.825 30) (width 0.2) (layer "F.Cu") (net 5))
 (segment (start 45.9359 29.5657) (end 45.2593 29.5657) (width 0.2) (layer "F.Cu") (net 5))
 (segment (start 41.205 33.62) (end 24 33.62) (width 0.2) (layer "F.Cu") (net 5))
 (segment (start 44.825 30) (end 41.205 33.62) (width 0.2) (layer "F.Cu") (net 5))
 (via (at 45.9359 29.5657) (size 0.6) (drill 0.3) (layers "F.Cu" "B.Cu") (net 5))
 (segment (start 58.8231 27.1671) (end 58.8231 33.62) (width 0.2) (layer "B.Cu") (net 5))
 (segment (start 50 22.62) (end 50 25.5016) (width 0.2) (layer "B.Cu") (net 5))
 (segment (start 50.2685 67.4683) (end 52.5485 65.1883) (width 0.2) (layer "B.Cu") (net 5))
 (segment (start 76 33.62) (end 74.8483 33.62) (width 0.2) (layer "B.Cu") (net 5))
 (segment (start 50 22.62) (end 48.7732 21.3932) (width 0.2) (layer "B.Cu") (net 5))
 (segment (start 58.8231 40.3769) (end 57.74 41.46) (width 0.2) (layer "B.Cu") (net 5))
 (segment (start 50 25.5016) (end 45.9359 29.5657) (width 0.2) (layer "B.Cu") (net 5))
 (segment (start 58.8231 33.62) (end 74.8483 33.62) (width 0.2) (layer "B.Cu") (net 5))
 (segment (start 49.475 18.9102) (end 50.5662 18.9102) (width 0.2) (layer "B.Cu") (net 5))
 (segment (start 58.8231 33.62) (end 58.8231 40.3769) (width 0.2) (layer "B.Cu") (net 5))
 (segment (start 52.5485 46.6515) (end 57.74 41.46) (width 0.2) (layer "B.Cu") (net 5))
 (segment (start 50.5662 18.9102) (end 58.8231 27.1671) (width 0.2) (layer "B.Cu") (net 5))
 (segment (start 52.5485 65.1883) (end 52.5485 46.6515) (width 0.2) (layer "B.Cu") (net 5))
 (segment (start 50 68.62) (end 50 67.4683) (width 0.2) (layer "B.Cu") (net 5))
 (segment (start 50 67.4683) (end 50.2685 67.4683) (width 0.2) (layer "B.Cu") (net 5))
 (segment (start 48.7732 19.612) (end 49.475 18.9102) (width 0.2) (layer "B.Cu") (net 5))
 (segment (start 48.7732 21.3932) (end 48.7732 19.612) (width 0.2) (layer "B.Cu") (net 5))
 (segment (start 57.74 51.62) (end 58.575 51.62) (width 0.2) (layer "F.Cu") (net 1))
 (segment (start 41.665 41.46) (end 42.5 41.46) (width 0.2) (layer "F.Cu") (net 10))
 (segment (start 41.665 44) (end 42.5 44) (width 0.2) (layer "F.Cu") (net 11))
 (segment (start 57.74 49.08) (end 58.575 49.08) (width 0.2) (layer "F.Cu") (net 2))
 (segment (start 57.74 46.54) (end 58.575 46.54) (width 0.2) (layer "F.Cu") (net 3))
 (segment (start 57.74 44) (end 58.575 44) (width 0.2) (layer "F.Cu") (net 4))
 (segment (start 57.74 36.38) (end 58.575 36.38) (width 0.2) (layer "F.Cu") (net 7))
 (segment (start 41.665 36.38) (end 42.5 36.38) (width 0.2) (layer "F.Cu") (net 8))
 (segment (start 41.665 38.92) (end 42.5 38.92) (width 0.2) (layer "F.Cu") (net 9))
 (segment (start 24 59.0083) (end 24.2879 59.0083) (width 0.2) (layer "B.Cu") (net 21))
 (segment (start 62.2121 16.3638) (end 62.8483 17) (width 0.2) (layer "B.Cu") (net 21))
 (segment (start 64 17) (end 62.8483 17) (width 0.2) (layer "B.Cu") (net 21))
 (segment (start 24.2879 59.0083) (end 36.8099 46.4863) (width 0.2) (layer "B.Cu") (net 21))
 (segment (start 24 60.16) (end 24 59.0083) (width 0.2) (layer "B.Cu") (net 21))
 (segment (start 36.8099 46.4863) (end 36.8099 29.0648) (width 0.2) (layer "B.Cu") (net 21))
 (segment (start 49.5109 16.3638) (end 62.2121 16.3638) (width 0.2) (layer "B.Cu") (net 21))
 (segment (start 36.8099 29.0648) (end 49.5109 16.3638) (width 0.2) (layer "B.Cu") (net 21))
 (segment (start 22.4073 33.7074) (end 36.5099 47.81) (width 0.2) (layer "F.Cu") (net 14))
 (segment (start 41.665 51.62) (end 42.5 51.62) (width 0.2) (layer "F.Cu") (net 14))
 (segment (start 43.5981 50.5219) (end 42.5 51.62) (width 0.2) (layer "F.Cu") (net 14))
 (segment (start 22.4073 25.4541) (end 22.4073 33.7074) (width 0.2) (layer "F.Cu") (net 14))
 (segment (start 30.8614 17) (end 22.4073 25.4541) (width 0.2) (layer "F.Cu") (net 14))
 (segment (start 36.5099 47.81) (end 42.7641 47.81) (width 0.2) (layer "F.Cu") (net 14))
 (segment (start 43.5981 48.644) (end 43.5981 50.5219) (width 0.2) (layer "F.Cu") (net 14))
 (segment (start 42.7641 47.81) (end 43.5981 48.644) (width 0.2) (layer "F.Cu") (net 14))
 (segment (start 36 17) (end 30.8614 17) (width 0.2) (layer "F.Cu") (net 14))
 (segment (start 47.3347 16.5136) (end 48.8483 15) (width 0.2) (layer "F.Cu") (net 15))
 (segment (start 60.73 18.81) (end 64 22.08) (width 0.2) (layer "F.Cu") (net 15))
 (segment (start 46.8483 17) (end 47.3347 16.5136) (width 0.2) (layer "F.Cu") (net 15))
 (segment (start 49.631 18.81) (end 60.73 18.81) (width 0.2) (layer "F.Cu") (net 15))
 (segment (start 47.3347 16.5136) (end 49.631 18.81) (width 0.2) (layer "F.Cu") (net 15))
 (segment (start 40 17) (end 46.8483 17) (width 0.2) (layer "F.Cu") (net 15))
 (segment (start 50 15) (end 48.8483 15) (width 0.2) (layer "F.Cu") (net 15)))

